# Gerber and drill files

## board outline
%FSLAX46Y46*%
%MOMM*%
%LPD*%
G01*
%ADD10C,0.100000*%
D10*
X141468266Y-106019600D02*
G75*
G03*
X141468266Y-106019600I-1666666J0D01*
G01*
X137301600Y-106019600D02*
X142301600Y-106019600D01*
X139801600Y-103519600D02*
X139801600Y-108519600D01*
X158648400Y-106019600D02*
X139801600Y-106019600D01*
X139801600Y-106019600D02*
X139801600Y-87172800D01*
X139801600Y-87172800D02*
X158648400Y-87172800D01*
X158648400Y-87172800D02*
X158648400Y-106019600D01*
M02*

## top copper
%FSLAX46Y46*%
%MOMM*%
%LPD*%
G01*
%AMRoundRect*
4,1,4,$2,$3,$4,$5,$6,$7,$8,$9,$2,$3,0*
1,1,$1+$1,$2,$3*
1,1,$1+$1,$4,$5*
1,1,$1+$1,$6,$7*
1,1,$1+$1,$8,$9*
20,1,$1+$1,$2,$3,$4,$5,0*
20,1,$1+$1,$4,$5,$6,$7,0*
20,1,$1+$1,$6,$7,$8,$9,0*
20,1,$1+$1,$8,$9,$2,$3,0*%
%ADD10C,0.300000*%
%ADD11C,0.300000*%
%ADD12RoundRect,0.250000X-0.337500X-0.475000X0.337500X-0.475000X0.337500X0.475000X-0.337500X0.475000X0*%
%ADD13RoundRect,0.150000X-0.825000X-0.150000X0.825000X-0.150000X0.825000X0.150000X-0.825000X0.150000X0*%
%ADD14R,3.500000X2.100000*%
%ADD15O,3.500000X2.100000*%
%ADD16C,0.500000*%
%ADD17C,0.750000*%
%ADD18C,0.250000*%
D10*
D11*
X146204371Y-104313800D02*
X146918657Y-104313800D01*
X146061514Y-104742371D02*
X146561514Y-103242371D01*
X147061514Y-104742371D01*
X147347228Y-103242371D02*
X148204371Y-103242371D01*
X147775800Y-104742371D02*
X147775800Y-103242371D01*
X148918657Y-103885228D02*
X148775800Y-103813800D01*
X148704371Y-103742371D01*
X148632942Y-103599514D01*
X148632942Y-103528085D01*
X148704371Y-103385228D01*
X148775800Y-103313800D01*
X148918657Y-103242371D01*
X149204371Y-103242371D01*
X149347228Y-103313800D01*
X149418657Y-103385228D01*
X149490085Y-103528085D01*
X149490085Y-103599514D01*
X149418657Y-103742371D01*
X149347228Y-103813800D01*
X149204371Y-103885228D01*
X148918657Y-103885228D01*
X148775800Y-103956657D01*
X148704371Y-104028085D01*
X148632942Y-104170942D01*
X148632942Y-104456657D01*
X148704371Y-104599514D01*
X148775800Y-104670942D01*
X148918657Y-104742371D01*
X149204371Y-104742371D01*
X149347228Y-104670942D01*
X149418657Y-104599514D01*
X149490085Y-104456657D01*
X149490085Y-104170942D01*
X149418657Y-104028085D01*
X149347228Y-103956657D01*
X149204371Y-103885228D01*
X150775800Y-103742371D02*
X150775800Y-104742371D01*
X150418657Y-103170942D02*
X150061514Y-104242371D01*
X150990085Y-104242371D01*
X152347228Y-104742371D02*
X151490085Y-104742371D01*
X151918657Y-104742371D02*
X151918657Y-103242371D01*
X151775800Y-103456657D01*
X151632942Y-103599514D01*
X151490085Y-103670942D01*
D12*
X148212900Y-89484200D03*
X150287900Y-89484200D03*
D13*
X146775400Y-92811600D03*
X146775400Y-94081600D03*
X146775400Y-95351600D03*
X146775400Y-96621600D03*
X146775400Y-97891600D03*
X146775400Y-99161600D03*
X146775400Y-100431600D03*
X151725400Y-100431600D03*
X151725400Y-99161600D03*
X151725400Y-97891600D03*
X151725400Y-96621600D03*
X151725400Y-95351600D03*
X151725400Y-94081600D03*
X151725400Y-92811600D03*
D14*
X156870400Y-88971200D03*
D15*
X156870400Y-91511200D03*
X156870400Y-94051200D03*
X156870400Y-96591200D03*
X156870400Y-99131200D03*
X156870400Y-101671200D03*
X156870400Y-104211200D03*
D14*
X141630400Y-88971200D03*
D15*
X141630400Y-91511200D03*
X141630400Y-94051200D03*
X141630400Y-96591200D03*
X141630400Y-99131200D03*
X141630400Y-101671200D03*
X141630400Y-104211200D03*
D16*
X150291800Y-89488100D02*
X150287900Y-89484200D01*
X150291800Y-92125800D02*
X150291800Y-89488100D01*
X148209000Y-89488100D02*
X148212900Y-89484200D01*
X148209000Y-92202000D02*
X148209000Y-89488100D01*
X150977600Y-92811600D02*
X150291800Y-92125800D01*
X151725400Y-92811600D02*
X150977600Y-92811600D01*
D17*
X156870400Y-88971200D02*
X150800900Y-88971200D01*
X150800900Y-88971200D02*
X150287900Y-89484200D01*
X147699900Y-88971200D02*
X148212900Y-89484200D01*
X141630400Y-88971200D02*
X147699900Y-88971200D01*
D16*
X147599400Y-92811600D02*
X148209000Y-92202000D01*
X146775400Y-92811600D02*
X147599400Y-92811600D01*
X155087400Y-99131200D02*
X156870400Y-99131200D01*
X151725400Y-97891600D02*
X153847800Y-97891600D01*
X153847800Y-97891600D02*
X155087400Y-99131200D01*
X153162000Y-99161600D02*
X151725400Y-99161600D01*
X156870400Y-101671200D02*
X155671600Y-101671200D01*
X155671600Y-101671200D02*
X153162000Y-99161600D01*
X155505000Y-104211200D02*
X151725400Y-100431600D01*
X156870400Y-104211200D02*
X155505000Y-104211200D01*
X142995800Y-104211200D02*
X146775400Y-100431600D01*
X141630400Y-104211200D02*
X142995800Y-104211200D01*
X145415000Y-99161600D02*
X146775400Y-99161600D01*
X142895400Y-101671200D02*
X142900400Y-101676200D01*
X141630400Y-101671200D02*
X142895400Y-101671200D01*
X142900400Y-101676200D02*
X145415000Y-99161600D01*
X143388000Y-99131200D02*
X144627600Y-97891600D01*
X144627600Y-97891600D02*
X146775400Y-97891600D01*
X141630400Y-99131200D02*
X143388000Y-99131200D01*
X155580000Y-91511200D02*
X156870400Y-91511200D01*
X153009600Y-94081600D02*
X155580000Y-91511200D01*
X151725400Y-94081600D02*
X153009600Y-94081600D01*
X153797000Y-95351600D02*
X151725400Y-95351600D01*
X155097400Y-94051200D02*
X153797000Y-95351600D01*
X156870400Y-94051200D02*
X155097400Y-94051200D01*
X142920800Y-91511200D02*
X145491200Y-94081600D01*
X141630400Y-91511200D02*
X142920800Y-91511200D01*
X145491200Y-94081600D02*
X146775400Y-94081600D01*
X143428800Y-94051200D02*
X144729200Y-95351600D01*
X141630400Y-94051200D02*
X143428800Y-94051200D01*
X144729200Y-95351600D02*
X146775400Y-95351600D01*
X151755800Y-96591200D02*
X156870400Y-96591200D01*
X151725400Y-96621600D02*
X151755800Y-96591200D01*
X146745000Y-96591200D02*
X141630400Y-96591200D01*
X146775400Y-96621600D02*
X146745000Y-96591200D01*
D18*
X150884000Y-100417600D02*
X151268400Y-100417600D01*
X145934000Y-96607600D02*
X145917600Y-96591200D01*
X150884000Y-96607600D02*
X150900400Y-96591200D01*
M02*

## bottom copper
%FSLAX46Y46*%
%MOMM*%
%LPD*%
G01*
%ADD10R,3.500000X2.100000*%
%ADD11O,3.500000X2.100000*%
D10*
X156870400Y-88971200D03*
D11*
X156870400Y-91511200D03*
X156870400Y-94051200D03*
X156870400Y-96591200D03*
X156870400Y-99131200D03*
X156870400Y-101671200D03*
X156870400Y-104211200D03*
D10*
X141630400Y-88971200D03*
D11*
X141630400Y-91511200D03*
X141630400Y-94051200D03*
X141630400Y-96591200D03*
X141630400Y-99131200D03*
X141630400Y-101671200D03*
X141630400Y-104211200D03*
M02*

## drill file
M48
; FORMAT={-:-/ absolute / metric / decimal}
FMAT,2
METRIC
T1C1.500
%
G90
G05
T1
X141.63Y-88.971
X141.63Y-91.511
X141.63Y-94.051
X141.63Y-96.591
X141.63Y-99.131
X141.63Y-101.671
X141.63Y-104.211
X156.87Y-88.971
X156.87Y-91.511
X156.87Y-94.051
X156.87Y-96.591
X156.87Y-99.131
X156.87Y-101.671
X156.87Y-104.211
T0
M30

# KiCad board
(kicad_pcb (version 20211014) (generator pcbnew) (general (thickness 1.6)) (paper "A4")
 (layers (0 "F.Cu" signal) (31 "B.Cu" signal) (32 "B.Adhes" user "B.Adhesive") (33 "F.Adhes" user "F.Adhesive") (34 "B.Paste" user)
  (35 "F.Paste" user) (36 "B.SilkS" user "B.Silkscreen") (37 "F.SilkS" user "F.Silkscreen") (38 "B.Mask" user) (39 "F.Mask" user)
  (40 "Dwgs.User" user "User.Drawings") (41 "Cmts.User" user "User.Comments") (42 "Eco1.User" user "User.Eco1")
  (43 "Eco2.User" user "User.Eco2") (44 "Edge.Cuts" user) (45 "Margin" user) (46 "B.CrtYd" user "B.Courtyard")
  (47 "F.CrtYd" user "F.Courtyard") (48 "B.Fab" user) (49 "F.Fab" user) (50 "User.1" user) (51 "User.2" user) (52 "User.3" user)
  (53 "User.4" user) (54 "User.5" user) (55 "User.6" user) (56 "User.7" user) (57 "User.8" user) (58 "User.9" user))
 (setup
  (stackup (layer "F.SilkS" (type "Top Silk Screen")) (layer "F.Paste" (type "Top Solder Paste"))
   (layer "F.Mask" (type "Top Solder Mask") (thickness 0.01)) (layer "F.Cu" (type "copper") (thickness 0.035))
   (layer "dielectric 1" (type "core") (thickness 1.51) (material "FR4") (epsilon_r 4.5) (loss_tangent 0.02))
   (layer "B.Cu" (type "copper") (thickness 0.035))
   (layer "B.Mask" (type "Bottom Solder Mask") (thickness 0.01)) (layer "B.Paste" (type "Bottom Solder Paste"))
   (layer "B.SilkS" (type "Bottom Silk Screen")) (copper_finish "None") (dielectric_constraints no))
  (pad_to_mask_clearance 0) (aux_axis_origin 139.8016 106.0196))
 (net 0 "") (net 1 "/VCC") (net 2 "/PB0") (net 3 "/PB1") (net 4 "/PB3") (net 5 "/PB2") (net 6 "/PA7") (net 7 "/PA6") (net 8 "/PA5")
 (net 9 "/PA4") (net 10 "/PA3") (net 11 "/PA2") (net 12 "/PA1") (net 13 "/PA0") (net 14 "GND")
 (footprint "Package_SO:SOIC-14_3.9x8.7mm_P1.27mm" (layer "F.Cu") (at 149.2504 96.6216)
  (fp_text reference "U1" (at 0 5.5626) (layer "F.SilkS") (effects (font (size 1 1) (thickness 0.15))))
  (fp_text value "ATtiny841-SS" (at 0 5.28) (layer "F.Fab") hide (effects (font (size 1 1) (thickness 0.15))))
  (pad "1" smd roundrect locked (at -2.475 -3.81) (size 1.95 0.6) (layers "F.Cu" "F.Paste" "F.Mask") (roundrect_rratio 0.25) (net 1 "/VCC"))
  (pad "2" smd roundrect locked (at -2.475 -2.54) (size 1.95 0.6) (layers "F.Cu" "F.Paste" "F.Mask") (roundrect_rratio 0.25) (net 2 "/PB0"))
  (pad "3" smd roundrect locked (at -2.475 -1.27) (size 1.95 0.6) (layers "F.Cu" "F.Paste" "F.Mask") (roundrect_rratio 0.25) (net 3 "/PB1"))
  (pad "4" smd roundrect locked (at -2.475 0) (size 1.95 0.6) (layers "F.Cu" "F.Paste" "F.Mask") (roundrect_rratio 0.25) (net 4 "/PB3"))
  (pad "5" smd roundrect locked (at -2.475 1.27) (size 1.95 0.6) (layers "F.Cu" "F.Paste" "F.Mask") (roundrect_rratio 0.25) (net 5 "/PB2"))
  (pad "6" smd roundrect locked (at -2.475 2.54) (size 1.95 0.6) (layers "F.Cu" "F.Paste" "F.Mask") (roundrect_rratio 0.25) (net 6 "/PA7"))
  (pad "7" smd roundrect locked (at -2.475 3.81) (size 1.95 0.6) (layers "F.Cu" "F.Paste" "F.Mask") (roundrect_rratio 0.25) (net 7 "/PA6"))
  (pad "8" smd roundrect locked (at 2.475 3.81) (size 1.95 0.6) (layers "F.Cu" "F.Paste" "F.Mask") (roundrect_rratio 0.25) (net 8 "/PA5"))
  (pad "9" smd roundrect locked (at 2.475 2.54) (size 1.95 0.6) (layers "F.Cu" "F.Paste" "F.Mask") (roundrect_rratio 0.25) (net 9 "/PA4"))
  (pad "10" smd roundrect locked (at 2.475 1.27) (size 1.95 0.6) (layers "F.Cu" "F.Paste" "F.Mask") (roundrect_rratio 0.25) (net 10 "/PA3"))
  (pad "11" smd roundrect locked (at 2.475 0) (size 1.95 0.6) (layers "F.Cu" "F.Paste" "F.Mask") (roundrect_rratio 0.25) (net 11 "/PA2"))
  (pad "12" smd roundrect locked (at 2.475 -1.27) (size 1.95 0.6) (layers "F.Cu" "F.Paste" "F.Mask") (roundrect_rratio 0.25) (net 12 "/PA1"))
  (pad "13" smd roundrect locked (at 2.475 -2.54) (size 1.95 0.6) (layers "F.Cu" "F.Paste" "F.Mask") (roundrect_rratio 0.25) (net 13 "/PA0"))
  (pad "14" smd roundrect locked (at 2.475 -3.81) (size 1.95 0.6) (layers "F.Cu" "F.Paste" "F.Mask") (roundrect_rratio 0.25) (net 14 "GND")))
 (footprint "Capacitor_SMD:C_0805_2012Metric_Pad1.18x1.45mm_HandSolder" (layer "F.Cu") (at 149.2504 89.4842)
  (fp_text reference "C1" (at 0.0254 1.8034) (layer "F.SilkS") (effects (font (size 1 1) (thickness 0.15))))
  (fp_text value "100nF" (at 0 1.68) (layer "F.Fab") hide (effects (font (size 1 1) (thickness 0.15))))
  (pad "1" smd roundrect locked (at -1.0375 0) (size 1.175 1.45) (layers "F.Cu" "F.Paste" "F.Mask") (roundrect_rratio 0.2127659574)
   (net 1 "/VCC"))
  (pad "2" smd roundrect locked (at 1.0375 0) (size 1.175 1.45) (layers "F.Cu" "F.Paste" "F.Mask") (roundrect_rratio 0.2127659574)
   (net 14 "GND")))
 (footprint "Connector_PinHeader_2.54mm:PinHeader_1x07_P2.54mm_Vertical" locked (layer "B.Cu") (at 156.8704 88.9712 180)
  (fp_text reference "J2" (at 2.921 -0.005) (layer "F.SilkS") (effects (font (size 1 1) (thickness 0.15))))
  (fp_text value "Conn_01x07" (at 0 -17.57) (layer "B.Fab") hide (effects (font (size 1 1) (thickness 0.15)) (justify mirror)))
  (pad "1" thru_hole rect locked (at 0 0 180) (size 3.5 2.1) (drill 1.5) (layers *.Cu *.Mask) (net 14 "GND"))
  (pad "2" thru_hole oval locked (at 0 -2.54 180) (size 3.5 2.1) (drill 1.5) (layers *.Cu *.Mask) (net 13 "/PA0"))
  (pad "3" thru_hole oval locked (at 0 -5.08 180) (size 3.5 2.1) (drill 1.5) (layers *.Cu *.Mask) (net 12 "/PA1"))
  (pad "4" thru_hole oval locked (at 0 -7.62 180) (size 3.5 2.1) (drill 1.5) (layers *.Cu *.Mask) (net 11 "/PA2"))
  (pad "5" thru_hole oval locked (at 0 -10.16 180) (size 3.5 2.1) (drill 1.5) (layers *.Cu *.Mask) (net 10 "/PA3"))
  (pad "6" thru_hole oval locked (at 0 -12.7 180) (size 3.5 2.1) (drill 1.5) (layers *.Cu *.Mask) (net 9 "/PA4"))
  (pad "7" thru_hole oval locked (at 0 -15.24 180) (size 3.5 2.1) (drill 1.5) (layers *.Cu *.Mask) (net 8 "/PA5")))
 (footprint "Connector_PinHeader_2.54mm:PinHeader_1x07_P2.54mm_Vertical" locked (layer "B.Cu") (at 141.6304 88.9712 180)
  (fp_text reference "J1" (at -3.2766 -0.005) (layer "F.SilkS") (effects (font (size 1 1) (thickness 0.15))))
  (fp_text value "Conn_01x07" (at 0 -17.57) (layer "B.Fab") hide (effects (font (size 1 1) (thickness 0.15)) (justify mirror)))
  (pad "1" thru_hole rect locked (at 0 0 180) (size 3.5 2.1) (drill 1.5) (layers *.Cu *.Mask) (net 1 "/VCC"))
  (pad "2" thru_hole oval locked (at 0 -2.54 180) (size 3.5 2.1) (drill 1.5) (layers *.Cu *.Mask) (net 2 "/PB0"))
  (pad "3" thru_hole oval locked (at 0 -5.08 180) (size 3.5 2.1) (drill 1.5) (layers *.Cu *.Mask) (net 3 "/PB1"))
  (pad "4" thru_hole oval locked (at 0 -7.62 180) (size 3.5 2.1) (drill 1.5) (layers *.Cu *.Mask) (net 4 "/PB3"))
  (pad "5" thru_hole oval locked (at 0 -10.16 180) (size 3.5 2.1) (drill 1.5) (layers *.Cu *.Mask) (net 5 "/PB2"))
  (pad "6" thru_hole oval locked (at 0 -12.7 180) (size 3.5 2.1) (drill 1.5) (layers *.Cu *.Mask) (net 6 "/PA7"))
  (pad "7" thru_hole oval locked (at 0 -15.24 180) (size 3.5 2.1) (drill 1.5) (layers *.Cu *.Mask) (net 7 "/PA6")))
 (gr_rect (start 158.6484 106.0196) (end 139.8016 87.1728) (layer "Edge.Cuts") (width 0.1) (fill none))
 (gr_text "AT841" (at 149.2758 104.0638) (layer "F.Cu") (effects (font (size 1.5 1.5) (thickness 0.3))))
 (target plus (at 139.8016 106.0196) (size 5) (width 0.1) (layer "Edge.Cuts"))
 (segment (start 148.209 92.202) (end 148.209 89.4881) (width 0.5) (layer "F.Cu") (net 1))
 (segment (start 148.209 89.4881) (end 148.2129 89.4842) (width 0.5) (layer "F.Cu") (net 1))
 (segment (start 146.7754 92.8116) (end 147.5994 92.8116) (width 0.5) (layer "F.Cu") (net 1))
 (segment (start 147.6999 88.9712) (end 148.2129 89.4842) (width 0.75) (layer "F.Cu") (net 1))
 (segment (start 141.6304 88.9712) (end 147.6999 88.9712) (width 0.75) (layer "F.Cu") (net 1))
 (segment (start 147.5994 92.8116) (end 148.209 92.202) (width 0.5) (layer "F.Cu") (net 1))
 (segment (start 145.4912 94.0816) (end 146.7754 94.0816) (width 0.5) (layer "F.Cu") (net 2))
 (segment (start 142.9208 91.5112) (end 145.4912 94.0816) (width 0.5) (layer "F.Cu") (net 2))
 (segment (start 141.6304 91.5112) (end 142.9208 91.5112) (width 0.5) (layer "F.Cu") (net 2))
 (segment (start 144.7292 95.3516) (end 146.7754 95.3516) (width 0.5) (layer "F.Cu") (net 3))
 (segment (start 143.4288 94.0512) (end 144.7292 95.3516) (width 0.5) (layer "F.Cu") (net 3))
 (segment (start 141.6304 94.0512) (end 143.4288 94.0512) (width 0.5) (layer "F.Cu") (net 3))
 (segment (start 144.6276 97.8916) (end 146.7754 97.8916) (width 0.5) (layer "F.Cu") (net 5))
 (segment (start 141.6304 99.1312) (end 143.388 99.1312) (width 0.5) (layer "F.Cu") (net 5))
 (segment (start 143.388 99.1312) (end 144.6276 97.8916) (width 0.5) (layer "F.Cu") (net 5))
 (segment (start 146.7754 96.6216) (end 146.745 96.5912) (width 0.5) (layer "F.Cu") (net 4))
 (segment (start 145.934 96.6076) (end 145.9176 96.5912) (width 0.25) (layer "F.Cu") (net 4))
 (segment (start 146.745 96.5912) (end 141.6304 96.5912) (width 0.5) (layer "F.Cu") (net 4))
 (segment (start 145.415 99.1616) (end 146.7754 99.1616) (width 0.5) (layer "F.Cu") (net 6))
 (segment (start 141.6304 101.6712) (end 142.8954 101.6712) (width 0.5) (layer "F.Cu") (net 6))
 (segment (start 142.8954 101.6712) (end 142.9004 101.6762) (width 0.5) (layer "F.Cu") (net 6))
 (segment (start 142.9004 101.6762) (end 145.415 99.1616) (width 0.5) (layer "F.Cu") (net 6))
 (segment (start 141.6304 104.2112) (end 142.9958 104.2112) (width 0.5) (layer "F.Cu") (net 7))
 (segment (start 142.9958 104.2112) (end 146.7754 100.4316) (width 0.5) (layer "F.Cu") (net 7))
 (segment (start 150.2918 92.1258) (end 150.2918 89.4881) (width 0.5) (layer "F.Cu") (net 14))
 (segment (start 150.9776 92.8116) (end 150.2918 92.1258) (width 0.5) (layer "F.Cu") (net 14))
 (segment (start 150.8009 88.9712) (end 150.2879 89.4842) (width 0.75) (layer "F.Cu") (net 14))
 (segment (start 150.2918 89.4881) (end 150.2879 89.4842) (width 0.5) (layer "F.Cu") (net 14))
 (segment (start 156.8704 88.9712) (end 150.8009 88.9712) (width 0.75) (layer "F.Cu") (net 14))
 (segment (start 151.7254 92.8116) (end 150.9776 92.8116) (width 0.5) (layer "F.Cu") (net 14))
 (segment (start 151.7254 94.0816) (end 153.0096 94.0816) (width 0.5) (layer "F.Cu") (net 13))
 (segment (start 155.58 91.5112) (end 156.8704 91.5112) (width 0.5) (layer "F.Cu") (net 13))
 (segment (start 153.0096 94.0816) (end 155.58 91.5112) (width 0.5) (layer "F.Cu") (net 13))
 (segment (start 156.8704 94.0512) (end 155.0974 94.0512) (width 0.5) (layer "F.Cu") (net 12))
 (segment (start 155.0974 94.0512) (end 153.797 95.3516) (width 0.5) (layer "F.Cu") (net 12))
 (segment (start 153.797 95.3516) (end 151.7254 95.3516) (width 0.5) (layer "F.Cu") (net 12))
 (segment (start 150.884 96.6076) (end 150.9004 96.5912) (width 0.25) (layer "F.Cu") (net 11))
 (segment (start 151.7558 96.5912) (end 156.8704 96.5912) (width 0.5) (layer "F.Cu") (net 11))
 (segment (start 151.7254 96.6216) (end 151.7558 96.5912) (width 0.5) (layer "F.Cu") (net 11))
 (segment (start 155.0874 99.1312) (end 156.8704 99.1312) (width 0.5) (layer "F.Cu") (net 10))
 (segment (start 153.8478 97.8916) (end 155.0874 99.1312) (width 0.5) (layer "F.Cu") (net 10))
 (segment (start 151.7254 97.8916) (end 153.8478 97.8916) (width 0.5) (layer "F.Cu") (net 10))
 (segment (start 156.8704 101.6712) (end 155.6716 101.6712) (width 0.5) (layer "F.Cu") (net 9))
 (segment (start 155.6716 101.6712) (end 153.162 99.1616) (width 0.5) (layer "F.Cu") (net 9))
 (segment (start 153.162 99.1616) (end 151.7254 99.1616) (width 0.5) (layer "F.Cu") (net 9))
 (segment (start 150.884 100.4176) (end 151.2684 100.4176) (width 0.25) (layer "F.Cu") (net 8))
 (segment (start 155.505 104.2112) (end 151.7254 100.4316) (width 0.5) (layer "F.Cu") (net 8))
 (segment (start 156.8704 104.2112) (end 155.505 104.2112) (width 0.5) (layer "F.Cu") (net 8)))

